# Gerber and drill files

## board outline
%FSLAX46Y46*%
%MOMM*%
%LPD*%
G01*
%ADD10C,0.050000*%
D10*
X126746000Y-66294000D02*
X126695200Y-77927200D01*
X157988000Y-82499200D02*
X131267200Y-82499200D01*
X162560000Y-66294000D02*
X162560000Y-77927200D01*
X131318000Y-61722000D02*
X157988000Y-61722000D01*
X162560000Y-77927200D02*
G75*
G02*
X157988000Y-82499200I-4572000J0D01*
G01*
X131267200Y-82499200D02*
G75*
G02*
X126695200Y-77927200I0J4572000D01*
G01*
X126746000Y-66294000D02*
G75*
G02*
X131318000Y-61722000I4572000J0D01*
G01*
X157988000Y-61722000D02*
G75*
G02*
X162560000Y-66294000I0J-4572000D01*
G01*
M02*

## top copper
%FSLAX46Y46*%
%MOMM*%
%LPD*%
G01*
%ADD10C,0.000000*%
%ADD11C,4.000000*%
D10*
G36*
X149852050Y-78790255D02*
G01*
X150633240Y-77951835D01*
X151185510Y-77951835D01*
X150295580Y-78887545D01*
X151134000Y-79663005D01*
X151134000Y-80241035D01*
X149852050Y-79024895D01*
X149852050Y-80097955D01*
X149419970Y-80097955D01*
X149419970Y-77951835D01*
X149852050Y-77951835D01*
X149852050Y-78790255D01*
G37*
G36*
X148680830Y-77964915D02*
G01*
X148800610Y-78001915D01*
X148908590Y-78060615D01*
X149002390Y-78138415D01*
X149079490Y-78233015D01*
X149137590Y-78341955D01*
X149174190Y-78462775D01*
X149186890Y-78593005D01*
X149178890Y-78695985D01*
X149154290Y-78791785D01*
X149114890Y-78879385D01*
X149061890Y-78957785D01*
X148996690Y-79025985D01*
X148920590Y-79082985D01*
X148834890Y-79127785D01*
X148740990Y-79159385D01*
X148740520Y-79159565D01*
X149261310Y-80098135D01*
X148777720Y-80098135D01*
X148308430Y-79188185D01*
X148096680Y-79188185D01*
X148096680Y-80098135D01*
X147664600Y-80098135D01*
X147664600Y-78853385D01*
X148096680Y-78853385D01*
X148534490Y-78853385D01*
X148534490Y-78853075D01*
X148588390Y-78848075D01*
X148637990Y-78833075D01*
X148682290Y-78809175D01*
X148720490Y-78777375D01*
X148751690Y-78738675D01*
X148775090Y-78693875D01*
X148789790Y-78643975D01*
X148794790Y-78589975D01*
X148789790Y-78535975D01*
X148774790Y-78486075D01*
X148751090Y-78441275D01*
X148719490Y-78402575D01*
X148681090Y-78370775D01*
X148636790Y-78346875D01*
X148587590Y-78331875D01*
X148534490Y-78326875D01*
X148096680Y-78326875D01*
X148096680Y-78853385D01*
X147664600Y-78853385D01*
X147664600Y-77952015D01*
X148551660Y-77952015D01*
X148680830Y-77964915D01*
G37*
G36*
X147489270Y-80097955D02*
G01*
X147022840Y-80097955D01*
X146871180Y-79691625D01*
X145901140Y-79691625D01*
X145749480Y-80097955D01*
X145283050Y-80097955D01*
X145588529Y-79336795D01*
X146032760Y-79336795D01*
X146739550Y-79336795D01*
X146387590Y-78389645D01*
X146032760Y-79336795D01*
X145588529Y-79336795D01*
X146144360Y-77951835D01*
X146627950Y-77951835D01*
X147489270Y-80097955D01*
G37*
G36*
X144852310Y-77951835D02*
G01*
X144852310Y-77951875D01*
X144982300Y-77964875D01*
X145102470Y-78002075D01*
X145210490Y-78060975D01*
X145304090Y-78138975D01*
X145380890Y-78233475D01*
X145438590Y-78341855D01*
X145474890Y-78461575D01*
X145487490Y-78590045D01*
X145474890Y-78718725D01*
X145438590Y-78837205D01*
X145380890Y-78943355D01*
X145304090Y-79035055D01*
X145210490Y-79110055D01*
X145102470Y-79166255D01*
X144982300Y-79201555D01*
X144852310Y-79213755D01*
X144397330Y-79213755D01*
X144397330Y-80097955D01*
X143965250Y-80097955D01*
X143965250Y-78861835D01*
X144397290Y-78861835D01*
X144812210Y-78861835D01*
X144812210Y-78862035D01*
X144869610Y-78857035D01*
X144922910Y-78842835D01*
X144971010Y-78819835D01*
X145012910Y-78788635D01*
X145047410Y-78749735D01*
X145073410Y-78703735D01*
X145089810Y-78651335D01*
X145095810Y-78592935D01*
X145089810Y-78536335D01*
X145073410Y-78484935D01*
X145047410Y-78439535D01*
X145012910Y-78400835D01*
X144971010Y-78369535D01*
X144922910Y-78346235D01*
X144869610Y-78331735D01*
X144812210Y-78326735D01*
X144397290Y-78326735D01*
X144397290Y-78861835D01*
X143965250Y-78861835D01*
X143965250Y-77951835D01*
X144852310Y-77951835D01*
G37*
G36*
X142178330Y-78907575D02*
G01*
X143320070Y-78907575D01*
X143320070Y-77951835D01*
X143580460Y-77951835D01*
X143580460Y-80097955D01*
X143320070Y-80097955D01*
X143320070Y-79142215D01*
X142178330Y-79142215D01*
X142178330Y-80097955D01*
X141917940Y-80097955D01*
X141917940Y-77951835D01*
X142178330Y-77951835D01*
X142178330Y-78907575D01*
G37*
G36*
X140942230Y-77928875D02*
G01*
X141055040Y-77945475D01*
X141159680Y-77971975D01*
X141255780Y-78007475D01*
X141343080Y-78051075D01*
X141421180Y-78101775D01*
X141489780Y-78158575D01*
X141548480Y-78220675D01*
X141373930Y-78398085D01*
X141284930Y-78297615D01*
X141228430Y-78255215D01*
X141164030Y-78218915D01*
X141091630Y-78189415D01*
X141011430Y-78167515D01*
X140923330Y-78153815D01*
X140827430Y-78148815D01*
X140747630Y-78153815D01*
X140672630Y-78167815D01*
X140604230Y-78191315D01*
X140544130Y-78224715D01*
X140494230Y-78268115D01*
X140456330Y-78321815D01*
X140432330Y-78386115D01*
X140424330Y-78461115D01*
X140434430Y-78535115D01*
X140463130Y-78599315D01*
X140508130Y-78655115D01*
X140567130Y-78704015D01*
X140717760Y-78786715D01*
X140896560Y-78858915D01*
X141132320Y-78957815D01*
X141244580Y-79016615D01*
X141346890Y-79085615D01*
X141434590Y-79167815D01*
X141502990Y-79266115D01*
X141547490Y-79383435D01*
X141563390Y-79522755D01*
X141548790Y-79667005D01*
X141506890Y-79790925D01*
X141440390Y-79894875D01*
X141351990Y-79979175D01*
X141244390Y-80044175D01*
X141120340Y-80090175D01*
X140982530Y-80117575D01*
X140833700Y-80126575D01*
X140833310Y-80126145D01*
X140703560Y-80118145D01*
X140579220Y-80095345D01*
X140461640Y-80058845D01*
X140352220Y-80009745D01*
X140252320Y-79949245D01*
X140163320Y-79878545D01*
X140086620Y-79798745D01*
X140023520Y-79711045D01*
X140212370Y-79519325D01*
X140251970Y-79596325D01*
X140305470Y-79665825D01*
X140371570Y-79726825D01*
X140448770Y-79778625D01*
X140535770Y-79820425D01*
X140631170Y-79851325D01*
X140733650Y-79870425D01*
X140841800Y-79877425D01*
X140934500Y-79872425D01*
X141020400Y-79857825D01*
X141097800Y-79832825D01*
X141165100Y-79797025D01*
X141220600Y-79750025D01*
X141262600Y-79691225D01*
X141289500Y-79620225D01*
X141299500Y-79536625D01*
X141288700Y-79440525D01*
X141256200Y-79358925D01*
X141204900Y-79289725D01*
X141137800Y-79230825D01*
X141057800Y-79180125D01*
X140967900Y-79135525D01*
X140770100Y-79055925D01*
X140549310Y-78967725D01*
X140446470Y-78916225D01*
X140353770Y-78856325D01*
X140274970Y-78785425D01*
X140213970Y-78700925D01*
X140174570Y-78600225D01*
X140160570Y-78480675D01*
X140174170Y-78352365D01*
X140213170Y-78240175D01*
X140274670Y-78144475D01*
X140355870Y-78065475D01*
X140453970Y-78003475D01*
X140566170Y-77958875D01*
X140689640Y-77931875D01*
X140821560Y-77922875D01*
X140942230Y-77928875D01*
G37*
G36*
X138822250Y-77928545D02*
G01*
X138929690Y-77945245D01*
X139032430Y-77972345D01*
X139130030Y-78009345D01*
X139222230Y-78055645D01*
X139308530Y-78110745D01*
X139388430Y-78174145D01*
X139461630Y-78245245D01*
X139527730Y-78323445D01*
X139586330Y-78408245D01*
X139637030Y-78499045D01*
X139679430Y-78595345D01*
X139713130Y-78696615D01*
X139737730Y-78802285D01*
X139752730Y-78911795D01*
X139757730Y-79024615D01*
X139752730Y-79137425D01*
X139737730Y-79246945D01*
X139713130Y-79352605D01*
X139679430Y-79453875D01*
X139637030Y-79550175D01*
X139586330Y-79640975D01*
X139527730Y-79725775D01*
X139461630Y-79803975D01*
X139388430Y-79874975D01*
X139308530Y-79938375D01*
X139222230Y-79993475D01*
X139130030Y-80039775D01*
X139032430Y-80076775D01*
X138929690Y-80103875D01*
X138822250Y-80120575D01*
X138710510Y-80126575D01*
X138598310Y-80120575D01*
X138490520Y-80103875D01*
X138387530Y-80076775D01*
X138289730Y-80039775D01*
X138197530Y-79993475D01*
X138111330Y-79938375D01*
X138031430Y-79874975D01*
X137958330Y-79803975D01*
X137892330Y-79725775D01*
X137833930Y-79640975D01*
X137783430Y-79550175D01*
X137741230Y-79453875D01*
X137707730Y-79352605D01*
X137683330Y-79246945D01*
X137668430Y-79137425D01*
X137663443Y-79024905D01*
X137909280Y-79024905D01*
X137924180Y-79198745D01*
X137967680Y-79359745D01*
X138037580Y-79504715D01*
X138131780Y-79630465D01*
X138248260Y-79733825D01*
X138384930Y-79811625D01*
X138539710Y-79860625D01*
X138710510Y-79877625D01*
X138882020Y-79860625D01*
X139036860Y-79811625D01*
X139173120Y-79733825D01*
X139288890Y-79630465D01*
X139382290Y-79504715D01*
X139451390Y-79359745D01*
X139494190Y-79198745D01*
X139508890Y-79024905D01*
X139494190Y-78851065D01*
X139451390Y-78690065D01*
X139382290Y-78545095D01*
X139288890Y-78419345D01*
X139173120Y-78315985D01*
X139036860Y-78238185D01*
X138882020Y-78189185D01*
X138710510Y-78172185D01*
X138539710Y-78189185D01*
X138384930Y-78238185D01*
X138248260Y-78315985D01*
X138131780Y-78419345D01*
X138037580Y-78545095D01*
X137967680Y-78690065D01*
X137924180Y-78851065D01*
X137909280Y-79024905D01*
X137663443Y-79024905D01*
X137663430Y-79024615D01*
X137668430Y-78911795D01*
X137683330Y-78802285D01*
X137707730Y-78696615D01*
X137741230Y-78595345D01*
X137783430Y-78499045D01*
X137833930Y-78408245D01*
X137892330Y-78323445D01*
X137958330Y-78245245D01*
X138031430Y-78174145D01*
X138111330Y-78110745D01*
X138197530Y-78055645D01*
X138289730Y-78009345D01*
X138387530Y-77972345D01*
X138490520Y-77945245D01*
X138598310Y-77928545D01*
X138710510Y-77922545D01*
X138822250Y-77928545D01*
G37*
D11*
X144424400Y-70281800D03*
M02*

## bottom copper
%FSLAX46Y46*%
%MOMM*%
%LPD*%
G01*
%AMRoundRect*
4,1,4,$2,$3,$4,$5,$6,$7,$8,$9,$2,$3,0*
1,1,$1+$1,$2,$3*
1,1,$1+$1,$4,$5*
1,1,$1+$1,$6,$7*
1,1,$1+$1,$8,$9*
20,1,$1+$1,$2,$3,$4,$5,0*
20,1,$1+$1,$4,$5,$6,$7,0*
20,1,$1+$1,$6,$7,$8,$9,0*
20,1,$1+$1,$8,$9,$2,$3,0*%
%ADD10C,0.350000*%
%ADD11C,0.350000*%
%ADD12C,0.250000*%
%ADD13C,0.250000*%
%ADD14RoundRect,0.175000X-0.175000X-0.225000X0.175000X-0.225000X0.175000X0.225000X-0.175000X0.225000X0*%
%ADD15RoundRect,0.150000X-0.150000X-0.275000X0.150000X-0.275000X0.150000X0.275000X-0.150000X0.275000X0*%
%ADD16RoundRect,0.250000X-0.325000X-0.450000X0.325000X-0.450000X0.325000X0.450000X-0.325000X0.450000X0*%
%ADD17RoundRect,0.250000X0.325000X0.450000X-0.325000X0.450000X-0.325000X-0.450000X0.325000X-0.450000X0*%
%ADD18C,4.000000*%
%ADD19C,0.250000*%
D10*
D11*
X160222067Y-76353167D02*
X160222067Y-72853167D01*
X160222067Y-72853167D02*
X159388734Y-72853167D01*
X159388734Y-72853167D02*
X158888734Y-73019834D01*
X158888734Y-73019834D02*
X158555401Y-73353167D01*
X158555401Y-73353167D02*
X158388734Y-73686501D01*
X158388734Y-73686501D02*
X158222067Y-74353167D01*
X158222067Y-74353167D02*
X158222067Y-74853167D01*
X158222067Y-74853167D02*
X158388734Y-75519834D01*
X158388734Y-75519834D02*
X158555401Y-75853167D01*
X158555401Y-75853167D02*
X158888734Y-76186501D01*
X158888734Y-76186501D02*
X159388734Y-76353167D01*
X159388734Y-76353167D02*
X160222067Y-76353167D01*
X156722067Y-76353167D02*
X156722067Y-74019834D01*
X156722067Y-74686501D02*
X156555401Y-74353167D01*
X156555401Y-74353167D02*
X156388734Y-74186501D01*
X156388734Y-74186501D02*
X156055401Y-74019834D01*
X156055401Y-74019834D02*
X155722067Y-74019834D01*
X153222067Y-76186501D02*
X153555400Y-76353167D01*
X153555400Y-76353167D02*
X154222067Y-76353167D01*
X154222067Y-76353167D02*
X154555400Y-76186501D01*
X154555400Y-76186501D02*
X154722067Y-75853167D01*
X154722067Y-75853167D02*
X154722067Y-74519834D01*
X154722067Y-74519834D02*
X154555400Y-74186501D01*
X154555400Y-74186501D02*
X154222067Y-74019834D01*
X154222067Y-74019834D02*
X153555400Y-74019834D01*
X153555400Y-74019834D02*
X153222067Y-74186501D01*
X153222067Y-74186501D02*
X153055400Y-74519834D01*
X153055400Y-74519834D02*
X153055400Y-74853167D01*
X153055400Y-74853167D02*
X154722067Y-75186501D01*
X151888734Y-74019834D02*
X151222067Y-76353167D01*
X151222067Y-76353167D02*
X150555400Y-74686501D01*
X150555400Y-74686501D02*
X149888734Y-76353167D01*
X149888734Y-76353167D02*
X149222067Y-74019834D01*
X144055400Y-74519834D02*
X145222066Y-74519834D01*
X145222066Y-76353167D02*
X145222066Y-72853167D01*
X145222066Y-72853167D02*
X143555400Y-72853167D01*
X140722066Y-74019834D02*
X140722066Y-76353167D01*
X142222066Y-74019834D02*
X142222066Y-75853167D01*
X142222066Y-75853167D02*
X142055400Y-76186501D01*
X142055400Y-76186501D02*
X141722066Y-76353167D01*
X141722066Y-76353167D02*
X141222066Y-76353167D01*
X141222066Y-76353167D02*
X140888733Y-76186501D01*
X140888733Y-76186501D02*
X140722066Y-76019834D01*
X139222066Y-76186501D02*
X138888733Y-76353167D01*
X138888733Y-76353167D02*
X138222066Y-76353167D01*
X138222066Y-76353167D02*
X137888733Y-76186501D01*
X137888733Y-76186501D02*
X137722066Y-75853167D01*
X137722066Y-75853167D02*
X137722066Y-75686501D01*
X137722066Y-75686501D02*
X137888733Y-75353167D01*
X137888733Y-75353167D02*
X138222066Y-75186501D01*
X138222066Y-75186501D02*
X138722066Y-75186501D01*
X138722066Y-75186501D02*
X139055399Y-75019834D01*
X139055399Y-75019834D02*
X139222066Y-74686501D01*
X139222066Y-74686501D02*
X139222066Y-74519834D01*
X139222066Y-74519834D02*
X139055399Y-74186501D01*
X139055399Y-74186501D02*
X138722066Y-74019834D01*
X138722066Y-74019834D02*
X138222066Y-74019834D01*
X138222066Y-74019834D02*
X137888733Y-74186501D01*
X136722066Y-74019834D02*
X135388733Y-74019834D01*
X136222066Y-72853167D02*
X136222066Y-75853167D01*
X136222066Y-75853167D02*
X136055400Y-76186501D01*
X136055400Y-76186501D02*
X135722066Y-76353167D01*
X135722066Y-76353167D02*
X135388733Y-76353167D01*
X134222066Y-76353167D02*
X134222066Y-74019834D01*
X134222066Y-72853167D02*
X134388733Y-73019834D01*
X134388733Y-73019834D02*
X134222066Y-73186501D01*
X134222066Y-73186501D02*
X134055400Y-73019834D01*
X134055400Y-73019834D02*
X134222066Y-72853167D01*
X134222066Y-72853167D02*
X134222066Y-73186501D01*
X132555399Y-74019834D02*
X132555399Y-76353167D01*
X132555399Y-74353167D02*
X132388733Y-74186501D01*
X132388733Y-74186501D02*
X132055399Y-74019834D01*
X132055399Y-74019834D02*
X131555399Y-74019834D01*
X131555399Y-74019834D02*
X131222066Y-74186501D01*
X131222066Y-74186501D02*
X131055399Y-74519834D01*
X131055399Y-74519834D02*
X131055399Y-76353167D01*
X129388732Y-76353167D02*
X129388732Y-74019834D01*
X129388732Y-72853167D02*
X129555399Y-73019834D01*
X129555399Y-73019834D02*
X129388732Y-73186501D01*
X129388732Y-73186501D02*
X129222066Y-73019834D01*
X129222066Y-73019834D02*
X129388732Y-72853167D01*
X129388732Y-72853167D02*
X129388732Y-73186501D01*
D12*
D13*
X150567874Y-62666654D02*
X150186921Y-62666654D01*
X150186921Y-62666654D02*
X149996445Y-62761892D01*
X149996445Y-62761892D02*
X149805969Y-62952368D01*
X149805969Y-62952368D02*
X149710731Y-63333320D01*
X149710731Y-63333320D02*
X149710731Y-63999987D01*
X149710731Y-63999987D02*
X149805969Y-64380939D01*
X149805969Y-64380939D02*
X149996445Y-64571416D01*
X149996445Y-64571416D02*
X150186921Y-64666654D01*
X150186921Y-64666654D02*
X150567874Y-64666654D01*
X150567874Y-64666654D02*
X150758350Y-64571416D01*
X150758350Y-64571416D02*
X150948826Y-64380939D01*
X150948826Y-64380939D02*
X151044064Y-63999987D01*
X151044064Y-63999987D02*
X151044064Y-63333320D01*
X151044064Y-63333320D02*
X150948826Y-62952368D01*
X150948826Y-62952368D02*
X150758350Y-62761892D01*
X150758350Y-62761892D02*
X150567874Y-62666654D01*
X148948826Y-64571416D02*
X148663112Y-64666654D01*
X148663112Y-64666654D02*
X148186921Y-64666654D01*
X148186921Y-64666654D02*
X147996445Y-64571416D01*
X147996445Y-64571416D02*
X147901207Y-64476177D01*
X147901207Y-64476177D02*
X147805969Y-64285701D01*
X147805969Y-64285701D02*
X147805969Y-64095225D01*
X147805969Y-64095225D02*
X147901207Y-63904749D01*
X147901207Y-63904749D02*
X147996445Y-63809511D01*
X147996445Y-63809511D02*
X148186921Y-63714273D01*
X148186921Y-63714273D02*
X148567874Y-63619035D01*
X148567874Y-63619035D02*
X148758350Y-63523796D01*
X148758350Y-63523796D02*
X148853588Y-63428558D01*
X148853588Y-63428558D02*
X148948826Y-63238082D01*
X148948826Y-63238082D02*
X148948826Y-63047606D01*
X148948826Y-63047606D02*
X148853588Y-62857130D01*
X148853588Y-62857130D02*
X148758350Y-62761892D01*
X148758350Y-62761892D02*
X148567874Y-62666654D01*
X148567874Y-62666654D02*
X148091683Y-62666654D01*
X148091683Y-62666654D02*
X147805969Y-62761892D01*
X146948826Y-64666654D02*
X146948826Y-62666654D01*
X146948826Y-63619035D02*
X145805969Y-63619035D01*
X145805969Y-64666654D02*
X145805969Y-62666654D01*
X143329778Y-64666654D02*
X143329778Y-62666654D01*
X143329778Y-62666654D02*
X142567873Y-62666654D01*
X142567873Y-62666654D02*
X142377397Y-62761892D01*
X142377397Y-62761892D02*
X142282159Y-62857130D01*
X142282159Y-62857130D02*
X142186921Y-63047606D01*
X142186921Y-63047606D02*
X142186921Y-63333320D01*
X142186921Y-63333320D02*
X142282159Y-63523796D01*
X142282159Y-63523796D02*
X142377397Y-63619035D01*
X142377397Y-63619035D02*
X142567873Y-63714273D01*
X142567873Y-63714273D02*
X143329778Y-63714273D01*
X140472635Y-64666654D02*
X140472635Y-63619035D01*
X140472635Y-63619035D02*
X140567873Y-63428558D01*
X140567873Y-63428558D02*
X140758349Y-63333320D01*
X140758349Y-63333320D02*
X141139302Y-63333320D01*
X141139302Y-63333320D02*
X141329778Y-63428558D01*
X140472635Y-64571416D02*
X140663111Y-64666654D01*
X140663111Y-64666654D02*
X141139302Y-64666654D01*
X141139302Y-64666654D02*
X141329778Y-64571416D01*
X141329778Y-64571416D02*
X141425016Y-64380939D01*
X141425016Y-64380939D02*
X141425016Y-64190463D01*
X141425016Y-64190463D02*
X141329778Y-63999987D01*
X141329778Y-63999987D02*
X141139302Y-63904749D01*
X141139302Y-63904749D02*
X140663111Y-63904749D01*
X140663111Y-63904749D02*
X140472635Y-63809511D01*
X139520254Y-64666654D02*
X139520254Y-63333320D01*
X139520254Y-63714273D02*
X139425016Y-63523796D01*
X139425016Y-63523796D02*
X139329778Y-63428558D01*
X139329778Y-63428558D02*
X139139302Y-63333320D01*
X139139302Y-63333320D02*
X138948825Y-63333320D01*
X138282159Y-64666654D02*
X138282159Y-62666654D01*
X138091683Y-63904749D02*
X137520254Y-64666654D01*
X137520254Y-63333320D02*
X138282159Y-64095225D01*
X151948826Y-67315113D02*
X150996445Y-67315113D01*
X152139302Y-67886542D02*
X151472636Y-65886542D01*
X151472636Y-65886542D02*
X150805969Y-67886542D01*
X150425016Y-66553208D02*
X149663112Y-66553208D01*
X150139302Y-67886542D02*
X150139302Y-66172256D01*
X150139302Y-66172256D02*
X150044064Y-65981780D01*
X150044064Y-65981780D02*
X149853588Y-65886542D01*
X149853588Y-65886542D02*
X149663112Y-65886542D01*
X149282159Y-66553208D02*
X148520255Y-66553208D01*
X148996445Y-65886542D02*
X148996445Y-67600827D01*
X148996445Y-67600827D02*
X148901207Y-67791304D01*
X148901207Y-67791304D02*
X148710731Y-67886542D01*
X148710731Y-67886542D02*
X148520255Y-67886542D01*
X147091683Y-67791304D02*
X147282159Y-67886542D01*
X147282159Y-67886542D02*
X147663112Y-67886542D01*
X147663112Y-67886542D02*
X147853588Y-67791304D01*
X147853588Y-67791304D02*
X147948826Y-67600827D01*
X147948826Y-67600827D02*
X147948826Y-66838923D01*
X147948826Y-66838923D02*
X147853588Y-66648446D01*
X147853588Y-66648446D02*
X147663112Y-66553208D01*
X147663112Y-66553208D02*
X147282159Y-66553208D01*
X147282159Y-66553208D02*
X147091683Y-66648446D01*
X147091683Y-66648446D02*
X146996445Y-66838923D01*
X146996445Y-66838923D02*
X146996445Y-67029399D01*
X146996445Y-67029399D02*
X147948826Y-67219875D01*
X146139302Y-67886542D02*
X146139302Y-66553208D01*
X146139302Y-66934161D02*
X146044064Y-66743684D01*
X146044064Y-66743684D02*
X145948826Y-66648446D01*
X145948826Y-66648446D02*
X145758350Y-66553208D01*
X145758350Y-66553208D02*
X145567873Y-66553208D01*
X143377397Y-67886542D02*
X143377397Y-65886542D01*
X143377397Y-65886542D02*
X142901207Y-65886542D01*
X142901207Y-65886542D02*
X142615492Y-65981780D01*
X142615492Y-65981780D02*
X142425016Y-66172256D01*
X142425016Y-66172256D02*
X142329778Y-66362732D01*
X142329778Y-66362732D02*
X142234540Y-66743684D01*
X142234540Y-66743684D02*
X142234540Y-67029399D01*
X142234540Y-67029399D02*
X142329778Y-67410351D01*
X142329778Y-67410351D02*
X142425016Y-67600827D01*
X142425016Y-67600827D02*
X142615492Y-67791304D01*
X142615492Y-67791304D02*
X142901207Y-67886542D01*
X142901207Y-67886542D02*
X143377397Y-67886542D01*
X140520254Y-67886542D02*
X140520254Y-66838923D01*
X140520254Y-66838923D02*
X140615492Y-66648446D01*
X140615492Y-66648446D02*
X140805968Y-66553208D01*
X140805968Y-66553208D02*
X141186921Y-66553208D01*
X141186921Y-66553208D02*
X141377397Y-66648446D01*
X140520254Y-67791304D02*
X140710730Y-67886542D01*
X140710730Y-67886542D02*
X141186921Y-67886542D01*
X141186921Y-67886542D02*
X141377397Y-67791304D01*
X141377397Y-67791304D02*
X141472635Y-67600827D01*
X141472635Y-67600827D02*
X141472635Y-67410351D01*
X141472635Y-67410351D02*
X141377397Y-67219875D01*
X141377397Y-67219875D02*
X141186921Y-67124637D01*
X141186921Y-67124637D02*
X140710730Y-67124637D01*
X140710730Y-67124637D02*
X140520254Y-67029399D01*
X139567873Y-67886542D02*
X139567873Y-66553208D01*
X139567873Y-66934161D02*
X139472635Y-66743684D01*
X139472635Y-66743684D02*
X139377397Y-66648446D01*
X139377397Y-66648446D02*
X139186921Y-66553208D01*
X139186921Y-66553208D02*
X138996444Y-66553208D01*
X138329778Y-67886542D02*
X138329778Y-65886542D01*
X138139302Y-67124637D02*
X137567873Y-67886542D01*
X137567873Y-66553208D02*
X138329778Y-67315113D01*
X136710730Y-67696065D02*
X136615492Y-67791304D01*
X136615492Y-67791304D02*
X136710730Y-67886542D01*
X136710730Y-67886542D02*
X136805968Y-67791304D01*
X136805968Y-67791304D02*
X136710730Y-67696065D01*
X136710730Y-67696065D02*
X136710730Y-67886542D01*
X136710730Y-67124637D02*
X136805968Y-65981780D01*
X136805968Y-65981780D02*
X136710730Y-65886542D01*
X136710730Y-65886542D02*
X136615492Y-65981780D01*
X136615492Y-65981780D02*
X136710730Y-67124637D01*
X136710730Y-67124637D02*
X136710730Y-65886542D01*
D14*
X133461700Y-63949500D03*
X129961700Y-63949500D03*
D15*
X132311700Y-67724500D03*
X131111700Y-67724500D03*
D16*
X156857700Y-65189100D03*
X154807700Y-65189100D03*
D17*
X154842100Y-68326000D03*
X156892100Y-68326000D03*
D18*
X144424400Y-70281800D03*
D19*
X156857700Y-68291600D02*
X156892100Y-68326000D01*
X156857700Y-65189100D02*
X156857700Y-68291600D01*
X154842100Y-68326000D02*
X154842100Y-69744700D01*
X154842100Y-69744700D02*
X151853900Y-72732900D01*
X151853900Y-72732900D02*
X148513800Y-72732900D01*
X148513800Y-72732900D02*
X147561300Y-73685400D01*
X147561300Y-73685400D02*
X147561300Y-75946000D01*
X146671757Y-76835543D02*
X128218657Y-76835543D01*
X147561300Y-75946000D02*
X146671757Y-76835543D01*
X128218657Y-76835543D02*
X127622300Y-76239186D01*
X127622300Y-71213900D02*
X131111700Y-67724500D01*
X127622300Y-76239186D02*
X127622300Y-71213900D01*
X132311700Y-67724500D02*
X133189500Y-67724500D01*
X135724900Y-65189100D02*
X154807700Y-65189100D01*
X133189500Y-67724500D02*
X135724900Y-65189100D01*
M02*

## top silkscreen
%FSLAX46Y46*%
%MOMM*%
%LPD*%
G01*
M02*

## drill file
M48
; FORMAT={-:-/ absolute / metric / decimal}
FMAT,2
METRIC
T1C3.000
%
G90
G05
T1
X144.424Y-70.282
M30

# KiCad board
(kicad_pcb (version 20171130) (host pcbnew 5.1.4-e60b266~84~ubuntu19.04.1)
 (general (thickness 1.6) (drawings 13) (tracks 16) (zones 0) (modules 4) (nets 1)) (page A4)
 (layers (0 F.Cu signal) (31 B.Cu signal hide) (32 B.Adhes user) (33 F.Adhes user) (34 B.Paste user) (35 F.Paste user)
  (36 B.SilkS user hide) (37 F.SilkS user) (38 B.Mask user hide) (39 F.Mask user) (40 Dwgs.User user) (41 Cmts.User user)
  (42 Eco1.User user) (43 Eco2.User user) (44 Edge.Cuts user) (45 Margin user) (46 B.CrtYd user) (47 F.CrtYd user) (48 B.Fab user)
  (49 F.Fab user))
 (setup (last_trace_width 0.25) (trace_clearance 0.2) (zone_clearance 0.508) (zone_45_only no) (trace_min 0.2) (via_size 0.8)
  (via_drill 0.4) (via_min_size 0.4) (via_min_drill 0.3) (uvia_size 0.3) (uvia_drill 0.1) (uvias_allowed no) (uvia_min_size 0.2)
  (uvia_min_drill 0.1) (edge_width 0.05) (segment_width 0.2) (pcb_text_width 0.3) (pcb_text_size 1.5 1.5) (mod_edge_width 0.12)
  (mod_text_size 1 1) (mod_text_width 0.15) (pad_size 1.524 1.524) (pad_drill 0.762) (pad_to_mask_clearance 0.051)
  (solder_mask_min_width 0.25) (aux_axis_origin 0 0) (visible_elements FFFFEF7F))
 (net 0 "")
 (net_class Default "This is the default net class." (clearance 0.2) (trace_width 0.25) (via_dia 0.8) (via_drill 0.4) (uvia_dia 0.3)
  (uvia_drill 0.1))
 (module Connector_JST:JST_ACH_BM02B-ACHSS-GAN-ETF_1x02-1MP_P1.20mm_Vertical (layer B.Cu) (at 131.7117 65.8495)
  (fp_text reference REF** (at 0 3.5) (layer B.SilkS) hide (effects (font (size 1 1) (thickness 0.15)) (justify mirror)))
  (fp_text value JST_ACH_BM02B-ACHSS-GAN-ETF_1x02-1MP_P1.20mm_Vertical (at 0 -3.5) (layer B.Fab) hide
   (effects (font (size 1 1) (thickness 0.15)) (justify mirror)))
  (pad MP smd roundrect (at 1.75 -1.9) (size 0.7 0.8) (layers B.Cu B.Paste B.Mask) (roundrect_rratio 0.25))
  (pad MP smd roundrect (at -1.75 -1.9) (size 0.7 0.8) (layers B.Cu B.Paste B.Mask) (roundrect_rratio 0.25))
  (pad 2 smd roundrect (at 0.6 1.875) (size 0.6 0.85) (layers B.Cu B.Paste B.Mask) (roundrect_rratio 0.25))
  (pad 1 smd roundrect (at -0.6 1.875) (size 0.6 0.85) (layers B.Cu B.Paste B.Mask) (roundrect_rratio 0.25)))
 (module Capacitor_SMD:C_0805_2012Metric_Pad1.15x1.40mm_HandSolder (layer B.Cu) (at 155.8327 65.1891)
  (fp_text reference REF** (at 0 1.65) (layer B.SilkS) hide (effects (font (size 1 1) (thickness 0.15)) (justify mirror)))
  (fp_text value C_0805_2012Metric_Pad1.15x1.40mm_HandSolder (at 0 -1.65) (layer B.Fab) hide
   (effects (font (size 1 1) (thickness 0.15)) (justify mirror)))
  (pad 2 smd roundrect (at 1.025 0) (size 1.15 1.4) (layers B.Cu B.Paste B.Mask) (roundrect_rratio 0.217391))
  (pad 1 smd roundrect (at -1.025 0) (size 1.15 1.4) (layers B.Cu B.Paste B.Mask) (roundrect_rratio 0.217391)))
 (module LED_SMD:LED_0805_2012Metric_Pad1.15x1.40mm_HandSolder (layer B.Cu) (at 155.8671 68.326 180)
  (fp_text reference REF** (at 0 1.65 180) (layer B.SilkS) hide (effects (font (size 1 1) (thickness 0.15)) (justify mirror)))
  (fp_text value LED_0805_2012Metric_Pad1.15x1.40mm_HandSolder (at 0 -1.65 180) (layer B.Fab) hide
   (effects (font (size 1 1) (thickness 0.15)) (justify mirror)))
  (pad 2 smd roundrect (at 1.025 0 180) (size 1.15 1.4) (layers B.Cu B.Paste B.Mask) (roundrect_rratio 0.217391))
  (pad 1 smd roundrect (at -1.025 0 180) (size 1.15 1.4) (layers B.Cu B.Paste B.Mask) (roundrect_rratio 0.217391)))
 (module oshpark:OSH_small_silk (layer F.Cu) (at 144.4244 71.8312)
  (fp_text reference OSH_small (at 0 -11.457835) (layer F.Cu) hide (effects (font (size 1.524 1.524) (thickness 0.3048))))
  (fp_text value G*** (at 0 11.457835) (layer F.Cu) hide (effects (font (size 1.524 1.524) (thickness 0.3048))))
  (fp_poly
   (pts (xy 6.76111 6.120635) (xy 6.20884 6.120635) (xy 5.42765 6.959055) (xy 5.42765 6.120635) (xy 4.99557 6.120635) (xy 4.99557 8.266755)
    (xy 5.42765 8.266755) (xy 5.42765 7.193695) (xy 6.7096 8.409835) (xy 6.7096 7.831805) (xy 5.87118 7.056345) (xy 6.76111 6.120635))
   (layer F.Cu) (width 0))
  (fp_poly
   (pts (xy 4.31659 7.328185) (xy 4.11009 7.022185) (xy 3.67228 7.022185) (xy 3.67228 6.495675) (xy 4.11009 6.495675) (xy 4.16319 6.500675)
    (xy 4.21239 6.515675) (xy 4.25669 6.539575) (xy 4.29509 6.571375) (xy 4.32669 6.610075) (xy 4.35039 6.654875) (xy 4.36539 6.704775)
    (xy 4.37039 6.758775) (xy 4.36539 6.812775) (xy 4.35069 6.862675) (xy 4.32729 6.907475) (xy 4.29609 6.946175) (xy 4.25789 6.977975)
    (xy 4.21359 7.001875) (xy 4.16399 7.016875) (xy 4.11009 7.021875) (xy 4.11009 7.022185) (xy 4.31659 7.328185) (xy 4.41049 7.296585)
    (xy 4.49619 7.251785) (xy 4.57229 7.194785) (xy 4.63749 7.126585) (xy 4.69049 7.048185) (xy 4.72989 6.960585) (xy 4.75449 6.864785)
    (xy 4.76249 6.761805) (xy 4.74979 6.631575) (xy 4.71319 6.510755) (xy 4.65509 6.401815) (xy 4.57799 6.307215) (xy 4.48419 6.229415)
    (xy 4.37621 6.170715) (xy 4.25643 6.133715) (xy 4.12726 6.120815) (xy 3.2402 6.120815) (xy 3.2402 8.266935) (xy 3.67228 8.266935)
    (xy 3.67228 7.356985) (xy 3.88403 7.356985) (xy 4.35332 8.266935) (xy 4.83691 8.266935) (xy 4.31612 7.328365) (xy 4.31659 7.328185))
   (layer F.Cu) (width 0))
  (fp_poly
   (pts (xy 2.59844 8.266755) (xy 1.96319 6.558445) (xy 2.31515 7.505595) (xy 1.60836 7.505595) (xy 1.96319 6.558445) (xy 2.59844 8.266755)
    (xy 3.06487 8.266755) (xy 2.20355 6.120635) (xy 1.71996 6.120635) (xy 0.85865 8.266755) (xy 1.32508 8.266755) (xy 1.47674 7.860425)
    (xy 2.44678 7.860425) (xy 2.59844 8.266755))
   (layer F.Cu) (width 0))
  (fp_poly
   (pts (xy 0.42791 6.120635) (xy -0.02711 6.495535) (xy 0.38781 6.495535) (xy 0.44521 6.500535) (xy 0.49851 6.515035) (xy 0.54661 6.538335)
    (xy 0.58851 6.569635) (xy 0.62301 6.608335) (xy 0.64901 6.653735) (xy 0.66541 6.705135) (xy 0.67141 6.761735) (xy 0.66541 6.820135)
    (xy 0.64901 6.872535) (xy 0.62301 6.918535) (xy 0.58851 6.957435) (xy 0.54661 6.988635) (xy 0.49851 7.011635) (xy 0.44521 7.025835)
    (xy 0.38781 7.030835) (xy 0.38781 7.030635) (xy -0.02711 7.030635) (xy -0.02711 6.495535) (xy 0.42791 6.120635) (xy -0.45915 6.120635)
    (xy -0.45915 8.266755) (xy -0.02707 8.266755) (xy -0.02707 7.382555) (xy 0.42791 7.382555) (xy 0.5579 7.370355) (xy 0.67807 7.335055)
    (xy 0.78609 7.278855) (xy 0.87969 7.203855) (xy 0.95649 7.112155) (xy 1.01419 7.006005) (xy 1.05049 6.887525) (xy 1.06309 6.758845)
    (xy 1.05049 6.630375) (xy 1.01419 6.510655) (xy 0.95649 6.402275) (xy 0.87969 6.307775) (xy 0.78609 6.229775) (xy 0.67807 6.170875)
    (xy 0.5579 6.133675) (xy 0.42791 6.120675) (xy 0.42791 6.120635))
   (layer F.Cu) (width 0))
  (fp_poly
   (pts (xy -1.10433 6.120635) (xy -1.10433 7.076375) (xy -2.24607 7.076375) (xy -2.24607 6.120635) (xy -2.50646 6.120635)
    (xy -2.50646 8.266755) (xy -2.24607 8.266755) (xy -2.24607 7.311015) (xy -1.10433 7.311015) (xy -1.10433 8.266755)
    (xy -0.84394 8.266755) (xy -0.84394 6.120635) (xy -1.10433 6.120635))
   (layer F.Cu) (width 0))
  (fp_poly
   (pts (xy -3.5907 8.295375) (xy -3.44187 8.286375) (xy -3.30406 8.258975) (xy -3.18001 8.212975) (xy -3.07241 8.147975)
    (xy -2.98401 8.063675) (xy -2.91751 7.959725) (xy -2.87561 7.835805) (xy -2.86101 7.691555) (xy -2.87691 7.552235)
    (xy -2.92141 7.434915) (xy -2.98981 7.336615) (xy -3.07751 7.254415) (xy -3.17982 7.185415) (xy -3.29208 7.126615)
    (xy -3.52784 7.027715) (xy -3.70664 6.955515) (xy -3.85727 6.872815) (xy -3.91627 6.823915) (xy -3.96127 6.768115)
    (xy -3.98997 6.703915) (xy -4.00007 6.629915) (xy -3.99207 6.554915) (xy -3.96807 6.490615) (xy -3.93017 6.436915)
    (xy -3.88027 6.393515) (xy -3.82017 6.360115) (xy -3.75177 6.336615) (xy -3.67677 6.322615) (xy -3.59697 6.317615)
    (xy -3.50107 6.322615) (xy -3.41297 6.336315) (xy -3.33277 6.358215) (xy -3.26037 6.387715) (xy -3.19597 6.424015)
    (xy -3.13947 6.466415) (xy -3.05047 6.566885) (xy -2.87592 6.389475) (xy -2.93462 6.327375) (xy -3.00322 6.270575)
    (xy -3.08132 6.219875) (xy -3.16862 6.176275) (xy -3.26472 6.140775) (xy -3.36936 6.114275) (xy -3.48217 6.097675)
    (xy -3.60284 6.091675) (xy -3.73476 6.100675) (xy -3.85823 6.127675) (xy -3.97043 6.172275) (xy -4.06853 6.234275)
    (xy -4.14973 6.313275) (xy -4.21123 6.408975) (xy -4.25023 6.521165) (xy -4.26383 6.649475) (xy -4.24983 6.769025)
    (xy -4.21043 6.869725) (xy -4.14943 6.954225) (xy -4.07063 7.025125) (xy -3.97793 7.085025) (xy -3.87509 7.136525) (xy -3.6543 7.224725)
    (xy -3.4565 7.304325) (xy -3.3666 7.348925) (xy -3.2866 7.399625) (xy -3.2195 7.458525) (xy -3.1682 7.527725) (xy -3.1357 7.609325)
    (xy -3.1249 7.705425) (xy -3.1349 7.789025) (xy -3.1618 7.860025) (xy -3.2038 7.918825) (xy -3.2593 7.965825) (xy -3.3266 8.001625)
    (xy -3.404 8.026625) (xy -3.4899 8.041225) (xy -3.5826 8.046225) (xy -3.69075 8.039225) (xy -3.79323 8.020125) (xy -3.88863 7.989225)
    (xy -3.97563 7.947425) (xy -4.05283 7.895625) (xy -4.11893 7.834625) (xy -4.17243 7.765125) (xy -4.21203 7.688125)
    (xy -4.40088 7.879845) (xy -4.33778 7.967545) (xy -4.26108 8.047345) (xy -4.17208 8.118045) (xy -4.07218 8.178545)
    (xy -3.96276 8.227645) (xy -3.84518 8.264145) (xy -3.72084 8.286945) (xy -3.59109 8.294945) (xy -3.5907 8.295375))
   (layer F.Cu) (width 0))
  (fp_poly
   (pts (xy -5.71389 8.295375) (xy -5.71389 8.046425) (xy -5.88469 8.029425) (xy -6.03947 7.980425) (xy -6.17614 7.902625)
    (xy -6.29262 7.799265) (xy -6.38682 7.673515) (xy -6.45672 7.528545) (xy -6.50022 7.367545) (xy -6.51512 7.193705)
    (xy -6.50022 7.019865) (xy -6.45672 6.858865) (xy -6.38682 6.713895) (xy -6.29262 6.588145) (xy -6.17614 6.484785)
    (xy -6.03947 6.406985) (xy -5.88469 6.357985) (xy -5.71389 6.340985) (xy -5.54238 6.357985) (xy -5.38754 6.406985)
    (xy -5.25128 6.484785) (xy -5.13551 6.588145) (xy -5.04211 6.713895) (xy -4.97301 6.858865) (xy -4.93021 7.019865)
    (xy -4.91551 7.193705) (xy -4.93021 7.367545) (xy -4.97301 7.528545) (xy -5.04211 7.673515) (xy -5.13551 7.799265)
    (xy -5.25128 7.902625) (xy -5.38754 7.980425) (xy -5.54238 8.029425) (xy -5.71389 8.046425) (xy -5.71389 8.295375)
    (xy -5.60215 8.289375) (xy -5.49471 8.272675) (xy -5.39197 8.245575) (xy -5.29437 8.208575) (xy -5.20217 8.162275)
    (xy -5.11587 8.107175) (xy -5.03597 8.043775) (xy -4.96277 7.972775) (xy -4.89667 7.894575) (xy -4.83807 7.809775)
    (xy -4.78737 7.718975) (xy -4.74497 7.622675) (xy -4.71127 7.521405) (xy -4.68667 7.415745) (xy -4.67167 7.306225)
    (xy -4.66667 7.193415) (xy -4.67167 7.080595) (xy -4.68667 6.971085) (xy -4.71127 6.865415) (xy -4.74497 6.764145)
    (xy -4.78737 6.667845) (xy -4.83807 6.577045) (xy -4.89667 6.492245) (xy -4.96277 6.414045) (xy -5.03597 6.342945)
    (xy -5.11587 6.279545) (xy -5.20217 6.224445) (xy -5.29437 6.178145) (xy -5.39197 6.141145) (xy -5.49471 6.114045)
    (xy -5.60215 6.097345) (xy -5.71389 6.091345) (xy -5.82609 6.097345) (xy -5.93388 6.114045) (xy -6.03687 6.141145)
    (xy -6.13467 6.178145) (xy -6.22687 6.224445) (xy -6.31307 6.279545) (xy -6.39297 6.342945) (xy -6.46607 6.414045)
    (xy -6.53207 6.492245) (xy -6.59047 6.577045) (xy -6.64097 6.667845) (xy -6.68317 6.764145) (xy -6.71667 6.865415)
    (xy -6.74107 6.971085) (xy -6.75597 7.080595) (xy -6.76097 7.193415) (xy -6.75597 7.306225) (xy -6.74107 7.415745)
    (xy -6.71667 7.521405) (xy -6.68317 7.622675) (xy -6.64097 7.718975) (xy -6.59047 7.809775) (xy -6.53207 7.894575)
    (xy -6.46607 7.972775) (xy -6.39297 8.043775) (xy -6.31307 8.107175) (xy -6.22687 8.162275) (xy -6.13467 8.208575)
    (xy -6.03687 8.245575) (xy -5.93388 8.272675) (xy -5.82609 8.289375) (xy -5.71389 8.295375))
   (layer F.Cu) (width 0)))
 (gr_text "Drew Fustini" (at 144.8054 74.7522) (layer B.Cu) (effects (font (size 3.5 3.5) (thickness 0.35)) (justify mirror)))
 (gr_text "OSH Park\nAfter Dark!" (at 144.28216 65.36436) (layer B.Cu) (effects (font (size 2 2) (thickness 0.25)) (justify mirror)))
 (gr_line (start 126.746 66.294) (end 126.6952 77.9272) (layer Edge.Cuts) (width 0.05))
 (gr_line (start 157.988 82.4992) (end 131.2672 82.4992) (layer Edge.Cuts) (width 0.05))
 (gr_line (start 162.56 66.294) (end 162.56 77.9272) (layer Edge.Cuts) (width 0.05))
 (gr_line (start 131.318 61.722) (end 157.988 61.722) (layer Edge.Cuts) (width 0.05))
 (gr_arc (start 157.988 77.9272) (end 157.988 82.4992) (angle -90) (layer Edge.Cuts) (width 0.05))
 (gr_arc (start 131.2672 77.9272) (end 126.6952 77.9272) (angle -90) (layer Edge.Cuts) (width 0.05))
 (gr_arc (start 131.318 66.294) (end 131.318 61.722) (angle -90) (layer Edge.Cuts) (width 0.05))
 (gr_arc (start 157.988 66.294) (end 162.56 66.294) (angle -90) (layer Edge.Cuts) (width 0.05))
 (via (at 144.4244 70.2818) (size 4) (drill 3) (layers F.Cu B.Cu) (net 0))
 (segment (start 156.8577 68.2916) (end 156.8921 68.326) (width 0.25) (layer B.Cu) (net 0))
 (segment (start 156.8577 65.1891) (end 156.8577 68.2916) (width 0.25) (layer B.Cu) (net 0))
 (segment (start 154.8421 68.326) (end 154.8421 69.7447) (width 0.25) (layer B.Cu) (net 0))
 (segment (start 154.8421 69.7447) (end 151.8539 72.7329) (width 0.25) (layer B.Cu) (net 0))
 (segment (start 151.8539 72.7329) (end 148.5138 72.7329) (width 0.25) (layer B.Cu) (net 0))
 (segment (start 148.5138 72.7329) (end 147.5613 73.6854) (width 0.25) (layer B.Cu) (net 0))
 (segment (start 147.5613 73.6854) (end 147.5613 75.946) (width 0.25) (layer B.Cu) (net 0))
 (segment (start 146.671757 76.835543) (end 128.218657 76.835543) (width 0.25) (layer B.Cu) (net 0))
 (segment (start 147.5613 75.946) (end 146.671757 76.835543) (width 0.25) (layer B.Cu) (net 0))
 (segment (start 128.218657 76.835543) (end 127.6223 76.239186) (width 0.25) (layer B.Cu) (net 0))
 (segment (start 127.6223 71.2139) (end 131.1117 67.7245) (width 0.25) (layer B.Cu) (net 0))
 (segment (start 127.6223 76.239186) (end 127.6223 71.2139) (width 0.25) (layer B.Cu) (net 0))
 (segment (start 132.3117 67.7245) (end 133.1895 67.7245) (width 0.25) (layer B.Cu) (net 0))
 (segment (start 135.7249 65.1891) (end 154.8077 65.1891) (width 0.25) (layer B.Cu) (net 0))
 (segment (start 133.1895 67.7245) (end 135.7249 65.1891) (width 0.25) (layer B.Cu) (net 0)))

